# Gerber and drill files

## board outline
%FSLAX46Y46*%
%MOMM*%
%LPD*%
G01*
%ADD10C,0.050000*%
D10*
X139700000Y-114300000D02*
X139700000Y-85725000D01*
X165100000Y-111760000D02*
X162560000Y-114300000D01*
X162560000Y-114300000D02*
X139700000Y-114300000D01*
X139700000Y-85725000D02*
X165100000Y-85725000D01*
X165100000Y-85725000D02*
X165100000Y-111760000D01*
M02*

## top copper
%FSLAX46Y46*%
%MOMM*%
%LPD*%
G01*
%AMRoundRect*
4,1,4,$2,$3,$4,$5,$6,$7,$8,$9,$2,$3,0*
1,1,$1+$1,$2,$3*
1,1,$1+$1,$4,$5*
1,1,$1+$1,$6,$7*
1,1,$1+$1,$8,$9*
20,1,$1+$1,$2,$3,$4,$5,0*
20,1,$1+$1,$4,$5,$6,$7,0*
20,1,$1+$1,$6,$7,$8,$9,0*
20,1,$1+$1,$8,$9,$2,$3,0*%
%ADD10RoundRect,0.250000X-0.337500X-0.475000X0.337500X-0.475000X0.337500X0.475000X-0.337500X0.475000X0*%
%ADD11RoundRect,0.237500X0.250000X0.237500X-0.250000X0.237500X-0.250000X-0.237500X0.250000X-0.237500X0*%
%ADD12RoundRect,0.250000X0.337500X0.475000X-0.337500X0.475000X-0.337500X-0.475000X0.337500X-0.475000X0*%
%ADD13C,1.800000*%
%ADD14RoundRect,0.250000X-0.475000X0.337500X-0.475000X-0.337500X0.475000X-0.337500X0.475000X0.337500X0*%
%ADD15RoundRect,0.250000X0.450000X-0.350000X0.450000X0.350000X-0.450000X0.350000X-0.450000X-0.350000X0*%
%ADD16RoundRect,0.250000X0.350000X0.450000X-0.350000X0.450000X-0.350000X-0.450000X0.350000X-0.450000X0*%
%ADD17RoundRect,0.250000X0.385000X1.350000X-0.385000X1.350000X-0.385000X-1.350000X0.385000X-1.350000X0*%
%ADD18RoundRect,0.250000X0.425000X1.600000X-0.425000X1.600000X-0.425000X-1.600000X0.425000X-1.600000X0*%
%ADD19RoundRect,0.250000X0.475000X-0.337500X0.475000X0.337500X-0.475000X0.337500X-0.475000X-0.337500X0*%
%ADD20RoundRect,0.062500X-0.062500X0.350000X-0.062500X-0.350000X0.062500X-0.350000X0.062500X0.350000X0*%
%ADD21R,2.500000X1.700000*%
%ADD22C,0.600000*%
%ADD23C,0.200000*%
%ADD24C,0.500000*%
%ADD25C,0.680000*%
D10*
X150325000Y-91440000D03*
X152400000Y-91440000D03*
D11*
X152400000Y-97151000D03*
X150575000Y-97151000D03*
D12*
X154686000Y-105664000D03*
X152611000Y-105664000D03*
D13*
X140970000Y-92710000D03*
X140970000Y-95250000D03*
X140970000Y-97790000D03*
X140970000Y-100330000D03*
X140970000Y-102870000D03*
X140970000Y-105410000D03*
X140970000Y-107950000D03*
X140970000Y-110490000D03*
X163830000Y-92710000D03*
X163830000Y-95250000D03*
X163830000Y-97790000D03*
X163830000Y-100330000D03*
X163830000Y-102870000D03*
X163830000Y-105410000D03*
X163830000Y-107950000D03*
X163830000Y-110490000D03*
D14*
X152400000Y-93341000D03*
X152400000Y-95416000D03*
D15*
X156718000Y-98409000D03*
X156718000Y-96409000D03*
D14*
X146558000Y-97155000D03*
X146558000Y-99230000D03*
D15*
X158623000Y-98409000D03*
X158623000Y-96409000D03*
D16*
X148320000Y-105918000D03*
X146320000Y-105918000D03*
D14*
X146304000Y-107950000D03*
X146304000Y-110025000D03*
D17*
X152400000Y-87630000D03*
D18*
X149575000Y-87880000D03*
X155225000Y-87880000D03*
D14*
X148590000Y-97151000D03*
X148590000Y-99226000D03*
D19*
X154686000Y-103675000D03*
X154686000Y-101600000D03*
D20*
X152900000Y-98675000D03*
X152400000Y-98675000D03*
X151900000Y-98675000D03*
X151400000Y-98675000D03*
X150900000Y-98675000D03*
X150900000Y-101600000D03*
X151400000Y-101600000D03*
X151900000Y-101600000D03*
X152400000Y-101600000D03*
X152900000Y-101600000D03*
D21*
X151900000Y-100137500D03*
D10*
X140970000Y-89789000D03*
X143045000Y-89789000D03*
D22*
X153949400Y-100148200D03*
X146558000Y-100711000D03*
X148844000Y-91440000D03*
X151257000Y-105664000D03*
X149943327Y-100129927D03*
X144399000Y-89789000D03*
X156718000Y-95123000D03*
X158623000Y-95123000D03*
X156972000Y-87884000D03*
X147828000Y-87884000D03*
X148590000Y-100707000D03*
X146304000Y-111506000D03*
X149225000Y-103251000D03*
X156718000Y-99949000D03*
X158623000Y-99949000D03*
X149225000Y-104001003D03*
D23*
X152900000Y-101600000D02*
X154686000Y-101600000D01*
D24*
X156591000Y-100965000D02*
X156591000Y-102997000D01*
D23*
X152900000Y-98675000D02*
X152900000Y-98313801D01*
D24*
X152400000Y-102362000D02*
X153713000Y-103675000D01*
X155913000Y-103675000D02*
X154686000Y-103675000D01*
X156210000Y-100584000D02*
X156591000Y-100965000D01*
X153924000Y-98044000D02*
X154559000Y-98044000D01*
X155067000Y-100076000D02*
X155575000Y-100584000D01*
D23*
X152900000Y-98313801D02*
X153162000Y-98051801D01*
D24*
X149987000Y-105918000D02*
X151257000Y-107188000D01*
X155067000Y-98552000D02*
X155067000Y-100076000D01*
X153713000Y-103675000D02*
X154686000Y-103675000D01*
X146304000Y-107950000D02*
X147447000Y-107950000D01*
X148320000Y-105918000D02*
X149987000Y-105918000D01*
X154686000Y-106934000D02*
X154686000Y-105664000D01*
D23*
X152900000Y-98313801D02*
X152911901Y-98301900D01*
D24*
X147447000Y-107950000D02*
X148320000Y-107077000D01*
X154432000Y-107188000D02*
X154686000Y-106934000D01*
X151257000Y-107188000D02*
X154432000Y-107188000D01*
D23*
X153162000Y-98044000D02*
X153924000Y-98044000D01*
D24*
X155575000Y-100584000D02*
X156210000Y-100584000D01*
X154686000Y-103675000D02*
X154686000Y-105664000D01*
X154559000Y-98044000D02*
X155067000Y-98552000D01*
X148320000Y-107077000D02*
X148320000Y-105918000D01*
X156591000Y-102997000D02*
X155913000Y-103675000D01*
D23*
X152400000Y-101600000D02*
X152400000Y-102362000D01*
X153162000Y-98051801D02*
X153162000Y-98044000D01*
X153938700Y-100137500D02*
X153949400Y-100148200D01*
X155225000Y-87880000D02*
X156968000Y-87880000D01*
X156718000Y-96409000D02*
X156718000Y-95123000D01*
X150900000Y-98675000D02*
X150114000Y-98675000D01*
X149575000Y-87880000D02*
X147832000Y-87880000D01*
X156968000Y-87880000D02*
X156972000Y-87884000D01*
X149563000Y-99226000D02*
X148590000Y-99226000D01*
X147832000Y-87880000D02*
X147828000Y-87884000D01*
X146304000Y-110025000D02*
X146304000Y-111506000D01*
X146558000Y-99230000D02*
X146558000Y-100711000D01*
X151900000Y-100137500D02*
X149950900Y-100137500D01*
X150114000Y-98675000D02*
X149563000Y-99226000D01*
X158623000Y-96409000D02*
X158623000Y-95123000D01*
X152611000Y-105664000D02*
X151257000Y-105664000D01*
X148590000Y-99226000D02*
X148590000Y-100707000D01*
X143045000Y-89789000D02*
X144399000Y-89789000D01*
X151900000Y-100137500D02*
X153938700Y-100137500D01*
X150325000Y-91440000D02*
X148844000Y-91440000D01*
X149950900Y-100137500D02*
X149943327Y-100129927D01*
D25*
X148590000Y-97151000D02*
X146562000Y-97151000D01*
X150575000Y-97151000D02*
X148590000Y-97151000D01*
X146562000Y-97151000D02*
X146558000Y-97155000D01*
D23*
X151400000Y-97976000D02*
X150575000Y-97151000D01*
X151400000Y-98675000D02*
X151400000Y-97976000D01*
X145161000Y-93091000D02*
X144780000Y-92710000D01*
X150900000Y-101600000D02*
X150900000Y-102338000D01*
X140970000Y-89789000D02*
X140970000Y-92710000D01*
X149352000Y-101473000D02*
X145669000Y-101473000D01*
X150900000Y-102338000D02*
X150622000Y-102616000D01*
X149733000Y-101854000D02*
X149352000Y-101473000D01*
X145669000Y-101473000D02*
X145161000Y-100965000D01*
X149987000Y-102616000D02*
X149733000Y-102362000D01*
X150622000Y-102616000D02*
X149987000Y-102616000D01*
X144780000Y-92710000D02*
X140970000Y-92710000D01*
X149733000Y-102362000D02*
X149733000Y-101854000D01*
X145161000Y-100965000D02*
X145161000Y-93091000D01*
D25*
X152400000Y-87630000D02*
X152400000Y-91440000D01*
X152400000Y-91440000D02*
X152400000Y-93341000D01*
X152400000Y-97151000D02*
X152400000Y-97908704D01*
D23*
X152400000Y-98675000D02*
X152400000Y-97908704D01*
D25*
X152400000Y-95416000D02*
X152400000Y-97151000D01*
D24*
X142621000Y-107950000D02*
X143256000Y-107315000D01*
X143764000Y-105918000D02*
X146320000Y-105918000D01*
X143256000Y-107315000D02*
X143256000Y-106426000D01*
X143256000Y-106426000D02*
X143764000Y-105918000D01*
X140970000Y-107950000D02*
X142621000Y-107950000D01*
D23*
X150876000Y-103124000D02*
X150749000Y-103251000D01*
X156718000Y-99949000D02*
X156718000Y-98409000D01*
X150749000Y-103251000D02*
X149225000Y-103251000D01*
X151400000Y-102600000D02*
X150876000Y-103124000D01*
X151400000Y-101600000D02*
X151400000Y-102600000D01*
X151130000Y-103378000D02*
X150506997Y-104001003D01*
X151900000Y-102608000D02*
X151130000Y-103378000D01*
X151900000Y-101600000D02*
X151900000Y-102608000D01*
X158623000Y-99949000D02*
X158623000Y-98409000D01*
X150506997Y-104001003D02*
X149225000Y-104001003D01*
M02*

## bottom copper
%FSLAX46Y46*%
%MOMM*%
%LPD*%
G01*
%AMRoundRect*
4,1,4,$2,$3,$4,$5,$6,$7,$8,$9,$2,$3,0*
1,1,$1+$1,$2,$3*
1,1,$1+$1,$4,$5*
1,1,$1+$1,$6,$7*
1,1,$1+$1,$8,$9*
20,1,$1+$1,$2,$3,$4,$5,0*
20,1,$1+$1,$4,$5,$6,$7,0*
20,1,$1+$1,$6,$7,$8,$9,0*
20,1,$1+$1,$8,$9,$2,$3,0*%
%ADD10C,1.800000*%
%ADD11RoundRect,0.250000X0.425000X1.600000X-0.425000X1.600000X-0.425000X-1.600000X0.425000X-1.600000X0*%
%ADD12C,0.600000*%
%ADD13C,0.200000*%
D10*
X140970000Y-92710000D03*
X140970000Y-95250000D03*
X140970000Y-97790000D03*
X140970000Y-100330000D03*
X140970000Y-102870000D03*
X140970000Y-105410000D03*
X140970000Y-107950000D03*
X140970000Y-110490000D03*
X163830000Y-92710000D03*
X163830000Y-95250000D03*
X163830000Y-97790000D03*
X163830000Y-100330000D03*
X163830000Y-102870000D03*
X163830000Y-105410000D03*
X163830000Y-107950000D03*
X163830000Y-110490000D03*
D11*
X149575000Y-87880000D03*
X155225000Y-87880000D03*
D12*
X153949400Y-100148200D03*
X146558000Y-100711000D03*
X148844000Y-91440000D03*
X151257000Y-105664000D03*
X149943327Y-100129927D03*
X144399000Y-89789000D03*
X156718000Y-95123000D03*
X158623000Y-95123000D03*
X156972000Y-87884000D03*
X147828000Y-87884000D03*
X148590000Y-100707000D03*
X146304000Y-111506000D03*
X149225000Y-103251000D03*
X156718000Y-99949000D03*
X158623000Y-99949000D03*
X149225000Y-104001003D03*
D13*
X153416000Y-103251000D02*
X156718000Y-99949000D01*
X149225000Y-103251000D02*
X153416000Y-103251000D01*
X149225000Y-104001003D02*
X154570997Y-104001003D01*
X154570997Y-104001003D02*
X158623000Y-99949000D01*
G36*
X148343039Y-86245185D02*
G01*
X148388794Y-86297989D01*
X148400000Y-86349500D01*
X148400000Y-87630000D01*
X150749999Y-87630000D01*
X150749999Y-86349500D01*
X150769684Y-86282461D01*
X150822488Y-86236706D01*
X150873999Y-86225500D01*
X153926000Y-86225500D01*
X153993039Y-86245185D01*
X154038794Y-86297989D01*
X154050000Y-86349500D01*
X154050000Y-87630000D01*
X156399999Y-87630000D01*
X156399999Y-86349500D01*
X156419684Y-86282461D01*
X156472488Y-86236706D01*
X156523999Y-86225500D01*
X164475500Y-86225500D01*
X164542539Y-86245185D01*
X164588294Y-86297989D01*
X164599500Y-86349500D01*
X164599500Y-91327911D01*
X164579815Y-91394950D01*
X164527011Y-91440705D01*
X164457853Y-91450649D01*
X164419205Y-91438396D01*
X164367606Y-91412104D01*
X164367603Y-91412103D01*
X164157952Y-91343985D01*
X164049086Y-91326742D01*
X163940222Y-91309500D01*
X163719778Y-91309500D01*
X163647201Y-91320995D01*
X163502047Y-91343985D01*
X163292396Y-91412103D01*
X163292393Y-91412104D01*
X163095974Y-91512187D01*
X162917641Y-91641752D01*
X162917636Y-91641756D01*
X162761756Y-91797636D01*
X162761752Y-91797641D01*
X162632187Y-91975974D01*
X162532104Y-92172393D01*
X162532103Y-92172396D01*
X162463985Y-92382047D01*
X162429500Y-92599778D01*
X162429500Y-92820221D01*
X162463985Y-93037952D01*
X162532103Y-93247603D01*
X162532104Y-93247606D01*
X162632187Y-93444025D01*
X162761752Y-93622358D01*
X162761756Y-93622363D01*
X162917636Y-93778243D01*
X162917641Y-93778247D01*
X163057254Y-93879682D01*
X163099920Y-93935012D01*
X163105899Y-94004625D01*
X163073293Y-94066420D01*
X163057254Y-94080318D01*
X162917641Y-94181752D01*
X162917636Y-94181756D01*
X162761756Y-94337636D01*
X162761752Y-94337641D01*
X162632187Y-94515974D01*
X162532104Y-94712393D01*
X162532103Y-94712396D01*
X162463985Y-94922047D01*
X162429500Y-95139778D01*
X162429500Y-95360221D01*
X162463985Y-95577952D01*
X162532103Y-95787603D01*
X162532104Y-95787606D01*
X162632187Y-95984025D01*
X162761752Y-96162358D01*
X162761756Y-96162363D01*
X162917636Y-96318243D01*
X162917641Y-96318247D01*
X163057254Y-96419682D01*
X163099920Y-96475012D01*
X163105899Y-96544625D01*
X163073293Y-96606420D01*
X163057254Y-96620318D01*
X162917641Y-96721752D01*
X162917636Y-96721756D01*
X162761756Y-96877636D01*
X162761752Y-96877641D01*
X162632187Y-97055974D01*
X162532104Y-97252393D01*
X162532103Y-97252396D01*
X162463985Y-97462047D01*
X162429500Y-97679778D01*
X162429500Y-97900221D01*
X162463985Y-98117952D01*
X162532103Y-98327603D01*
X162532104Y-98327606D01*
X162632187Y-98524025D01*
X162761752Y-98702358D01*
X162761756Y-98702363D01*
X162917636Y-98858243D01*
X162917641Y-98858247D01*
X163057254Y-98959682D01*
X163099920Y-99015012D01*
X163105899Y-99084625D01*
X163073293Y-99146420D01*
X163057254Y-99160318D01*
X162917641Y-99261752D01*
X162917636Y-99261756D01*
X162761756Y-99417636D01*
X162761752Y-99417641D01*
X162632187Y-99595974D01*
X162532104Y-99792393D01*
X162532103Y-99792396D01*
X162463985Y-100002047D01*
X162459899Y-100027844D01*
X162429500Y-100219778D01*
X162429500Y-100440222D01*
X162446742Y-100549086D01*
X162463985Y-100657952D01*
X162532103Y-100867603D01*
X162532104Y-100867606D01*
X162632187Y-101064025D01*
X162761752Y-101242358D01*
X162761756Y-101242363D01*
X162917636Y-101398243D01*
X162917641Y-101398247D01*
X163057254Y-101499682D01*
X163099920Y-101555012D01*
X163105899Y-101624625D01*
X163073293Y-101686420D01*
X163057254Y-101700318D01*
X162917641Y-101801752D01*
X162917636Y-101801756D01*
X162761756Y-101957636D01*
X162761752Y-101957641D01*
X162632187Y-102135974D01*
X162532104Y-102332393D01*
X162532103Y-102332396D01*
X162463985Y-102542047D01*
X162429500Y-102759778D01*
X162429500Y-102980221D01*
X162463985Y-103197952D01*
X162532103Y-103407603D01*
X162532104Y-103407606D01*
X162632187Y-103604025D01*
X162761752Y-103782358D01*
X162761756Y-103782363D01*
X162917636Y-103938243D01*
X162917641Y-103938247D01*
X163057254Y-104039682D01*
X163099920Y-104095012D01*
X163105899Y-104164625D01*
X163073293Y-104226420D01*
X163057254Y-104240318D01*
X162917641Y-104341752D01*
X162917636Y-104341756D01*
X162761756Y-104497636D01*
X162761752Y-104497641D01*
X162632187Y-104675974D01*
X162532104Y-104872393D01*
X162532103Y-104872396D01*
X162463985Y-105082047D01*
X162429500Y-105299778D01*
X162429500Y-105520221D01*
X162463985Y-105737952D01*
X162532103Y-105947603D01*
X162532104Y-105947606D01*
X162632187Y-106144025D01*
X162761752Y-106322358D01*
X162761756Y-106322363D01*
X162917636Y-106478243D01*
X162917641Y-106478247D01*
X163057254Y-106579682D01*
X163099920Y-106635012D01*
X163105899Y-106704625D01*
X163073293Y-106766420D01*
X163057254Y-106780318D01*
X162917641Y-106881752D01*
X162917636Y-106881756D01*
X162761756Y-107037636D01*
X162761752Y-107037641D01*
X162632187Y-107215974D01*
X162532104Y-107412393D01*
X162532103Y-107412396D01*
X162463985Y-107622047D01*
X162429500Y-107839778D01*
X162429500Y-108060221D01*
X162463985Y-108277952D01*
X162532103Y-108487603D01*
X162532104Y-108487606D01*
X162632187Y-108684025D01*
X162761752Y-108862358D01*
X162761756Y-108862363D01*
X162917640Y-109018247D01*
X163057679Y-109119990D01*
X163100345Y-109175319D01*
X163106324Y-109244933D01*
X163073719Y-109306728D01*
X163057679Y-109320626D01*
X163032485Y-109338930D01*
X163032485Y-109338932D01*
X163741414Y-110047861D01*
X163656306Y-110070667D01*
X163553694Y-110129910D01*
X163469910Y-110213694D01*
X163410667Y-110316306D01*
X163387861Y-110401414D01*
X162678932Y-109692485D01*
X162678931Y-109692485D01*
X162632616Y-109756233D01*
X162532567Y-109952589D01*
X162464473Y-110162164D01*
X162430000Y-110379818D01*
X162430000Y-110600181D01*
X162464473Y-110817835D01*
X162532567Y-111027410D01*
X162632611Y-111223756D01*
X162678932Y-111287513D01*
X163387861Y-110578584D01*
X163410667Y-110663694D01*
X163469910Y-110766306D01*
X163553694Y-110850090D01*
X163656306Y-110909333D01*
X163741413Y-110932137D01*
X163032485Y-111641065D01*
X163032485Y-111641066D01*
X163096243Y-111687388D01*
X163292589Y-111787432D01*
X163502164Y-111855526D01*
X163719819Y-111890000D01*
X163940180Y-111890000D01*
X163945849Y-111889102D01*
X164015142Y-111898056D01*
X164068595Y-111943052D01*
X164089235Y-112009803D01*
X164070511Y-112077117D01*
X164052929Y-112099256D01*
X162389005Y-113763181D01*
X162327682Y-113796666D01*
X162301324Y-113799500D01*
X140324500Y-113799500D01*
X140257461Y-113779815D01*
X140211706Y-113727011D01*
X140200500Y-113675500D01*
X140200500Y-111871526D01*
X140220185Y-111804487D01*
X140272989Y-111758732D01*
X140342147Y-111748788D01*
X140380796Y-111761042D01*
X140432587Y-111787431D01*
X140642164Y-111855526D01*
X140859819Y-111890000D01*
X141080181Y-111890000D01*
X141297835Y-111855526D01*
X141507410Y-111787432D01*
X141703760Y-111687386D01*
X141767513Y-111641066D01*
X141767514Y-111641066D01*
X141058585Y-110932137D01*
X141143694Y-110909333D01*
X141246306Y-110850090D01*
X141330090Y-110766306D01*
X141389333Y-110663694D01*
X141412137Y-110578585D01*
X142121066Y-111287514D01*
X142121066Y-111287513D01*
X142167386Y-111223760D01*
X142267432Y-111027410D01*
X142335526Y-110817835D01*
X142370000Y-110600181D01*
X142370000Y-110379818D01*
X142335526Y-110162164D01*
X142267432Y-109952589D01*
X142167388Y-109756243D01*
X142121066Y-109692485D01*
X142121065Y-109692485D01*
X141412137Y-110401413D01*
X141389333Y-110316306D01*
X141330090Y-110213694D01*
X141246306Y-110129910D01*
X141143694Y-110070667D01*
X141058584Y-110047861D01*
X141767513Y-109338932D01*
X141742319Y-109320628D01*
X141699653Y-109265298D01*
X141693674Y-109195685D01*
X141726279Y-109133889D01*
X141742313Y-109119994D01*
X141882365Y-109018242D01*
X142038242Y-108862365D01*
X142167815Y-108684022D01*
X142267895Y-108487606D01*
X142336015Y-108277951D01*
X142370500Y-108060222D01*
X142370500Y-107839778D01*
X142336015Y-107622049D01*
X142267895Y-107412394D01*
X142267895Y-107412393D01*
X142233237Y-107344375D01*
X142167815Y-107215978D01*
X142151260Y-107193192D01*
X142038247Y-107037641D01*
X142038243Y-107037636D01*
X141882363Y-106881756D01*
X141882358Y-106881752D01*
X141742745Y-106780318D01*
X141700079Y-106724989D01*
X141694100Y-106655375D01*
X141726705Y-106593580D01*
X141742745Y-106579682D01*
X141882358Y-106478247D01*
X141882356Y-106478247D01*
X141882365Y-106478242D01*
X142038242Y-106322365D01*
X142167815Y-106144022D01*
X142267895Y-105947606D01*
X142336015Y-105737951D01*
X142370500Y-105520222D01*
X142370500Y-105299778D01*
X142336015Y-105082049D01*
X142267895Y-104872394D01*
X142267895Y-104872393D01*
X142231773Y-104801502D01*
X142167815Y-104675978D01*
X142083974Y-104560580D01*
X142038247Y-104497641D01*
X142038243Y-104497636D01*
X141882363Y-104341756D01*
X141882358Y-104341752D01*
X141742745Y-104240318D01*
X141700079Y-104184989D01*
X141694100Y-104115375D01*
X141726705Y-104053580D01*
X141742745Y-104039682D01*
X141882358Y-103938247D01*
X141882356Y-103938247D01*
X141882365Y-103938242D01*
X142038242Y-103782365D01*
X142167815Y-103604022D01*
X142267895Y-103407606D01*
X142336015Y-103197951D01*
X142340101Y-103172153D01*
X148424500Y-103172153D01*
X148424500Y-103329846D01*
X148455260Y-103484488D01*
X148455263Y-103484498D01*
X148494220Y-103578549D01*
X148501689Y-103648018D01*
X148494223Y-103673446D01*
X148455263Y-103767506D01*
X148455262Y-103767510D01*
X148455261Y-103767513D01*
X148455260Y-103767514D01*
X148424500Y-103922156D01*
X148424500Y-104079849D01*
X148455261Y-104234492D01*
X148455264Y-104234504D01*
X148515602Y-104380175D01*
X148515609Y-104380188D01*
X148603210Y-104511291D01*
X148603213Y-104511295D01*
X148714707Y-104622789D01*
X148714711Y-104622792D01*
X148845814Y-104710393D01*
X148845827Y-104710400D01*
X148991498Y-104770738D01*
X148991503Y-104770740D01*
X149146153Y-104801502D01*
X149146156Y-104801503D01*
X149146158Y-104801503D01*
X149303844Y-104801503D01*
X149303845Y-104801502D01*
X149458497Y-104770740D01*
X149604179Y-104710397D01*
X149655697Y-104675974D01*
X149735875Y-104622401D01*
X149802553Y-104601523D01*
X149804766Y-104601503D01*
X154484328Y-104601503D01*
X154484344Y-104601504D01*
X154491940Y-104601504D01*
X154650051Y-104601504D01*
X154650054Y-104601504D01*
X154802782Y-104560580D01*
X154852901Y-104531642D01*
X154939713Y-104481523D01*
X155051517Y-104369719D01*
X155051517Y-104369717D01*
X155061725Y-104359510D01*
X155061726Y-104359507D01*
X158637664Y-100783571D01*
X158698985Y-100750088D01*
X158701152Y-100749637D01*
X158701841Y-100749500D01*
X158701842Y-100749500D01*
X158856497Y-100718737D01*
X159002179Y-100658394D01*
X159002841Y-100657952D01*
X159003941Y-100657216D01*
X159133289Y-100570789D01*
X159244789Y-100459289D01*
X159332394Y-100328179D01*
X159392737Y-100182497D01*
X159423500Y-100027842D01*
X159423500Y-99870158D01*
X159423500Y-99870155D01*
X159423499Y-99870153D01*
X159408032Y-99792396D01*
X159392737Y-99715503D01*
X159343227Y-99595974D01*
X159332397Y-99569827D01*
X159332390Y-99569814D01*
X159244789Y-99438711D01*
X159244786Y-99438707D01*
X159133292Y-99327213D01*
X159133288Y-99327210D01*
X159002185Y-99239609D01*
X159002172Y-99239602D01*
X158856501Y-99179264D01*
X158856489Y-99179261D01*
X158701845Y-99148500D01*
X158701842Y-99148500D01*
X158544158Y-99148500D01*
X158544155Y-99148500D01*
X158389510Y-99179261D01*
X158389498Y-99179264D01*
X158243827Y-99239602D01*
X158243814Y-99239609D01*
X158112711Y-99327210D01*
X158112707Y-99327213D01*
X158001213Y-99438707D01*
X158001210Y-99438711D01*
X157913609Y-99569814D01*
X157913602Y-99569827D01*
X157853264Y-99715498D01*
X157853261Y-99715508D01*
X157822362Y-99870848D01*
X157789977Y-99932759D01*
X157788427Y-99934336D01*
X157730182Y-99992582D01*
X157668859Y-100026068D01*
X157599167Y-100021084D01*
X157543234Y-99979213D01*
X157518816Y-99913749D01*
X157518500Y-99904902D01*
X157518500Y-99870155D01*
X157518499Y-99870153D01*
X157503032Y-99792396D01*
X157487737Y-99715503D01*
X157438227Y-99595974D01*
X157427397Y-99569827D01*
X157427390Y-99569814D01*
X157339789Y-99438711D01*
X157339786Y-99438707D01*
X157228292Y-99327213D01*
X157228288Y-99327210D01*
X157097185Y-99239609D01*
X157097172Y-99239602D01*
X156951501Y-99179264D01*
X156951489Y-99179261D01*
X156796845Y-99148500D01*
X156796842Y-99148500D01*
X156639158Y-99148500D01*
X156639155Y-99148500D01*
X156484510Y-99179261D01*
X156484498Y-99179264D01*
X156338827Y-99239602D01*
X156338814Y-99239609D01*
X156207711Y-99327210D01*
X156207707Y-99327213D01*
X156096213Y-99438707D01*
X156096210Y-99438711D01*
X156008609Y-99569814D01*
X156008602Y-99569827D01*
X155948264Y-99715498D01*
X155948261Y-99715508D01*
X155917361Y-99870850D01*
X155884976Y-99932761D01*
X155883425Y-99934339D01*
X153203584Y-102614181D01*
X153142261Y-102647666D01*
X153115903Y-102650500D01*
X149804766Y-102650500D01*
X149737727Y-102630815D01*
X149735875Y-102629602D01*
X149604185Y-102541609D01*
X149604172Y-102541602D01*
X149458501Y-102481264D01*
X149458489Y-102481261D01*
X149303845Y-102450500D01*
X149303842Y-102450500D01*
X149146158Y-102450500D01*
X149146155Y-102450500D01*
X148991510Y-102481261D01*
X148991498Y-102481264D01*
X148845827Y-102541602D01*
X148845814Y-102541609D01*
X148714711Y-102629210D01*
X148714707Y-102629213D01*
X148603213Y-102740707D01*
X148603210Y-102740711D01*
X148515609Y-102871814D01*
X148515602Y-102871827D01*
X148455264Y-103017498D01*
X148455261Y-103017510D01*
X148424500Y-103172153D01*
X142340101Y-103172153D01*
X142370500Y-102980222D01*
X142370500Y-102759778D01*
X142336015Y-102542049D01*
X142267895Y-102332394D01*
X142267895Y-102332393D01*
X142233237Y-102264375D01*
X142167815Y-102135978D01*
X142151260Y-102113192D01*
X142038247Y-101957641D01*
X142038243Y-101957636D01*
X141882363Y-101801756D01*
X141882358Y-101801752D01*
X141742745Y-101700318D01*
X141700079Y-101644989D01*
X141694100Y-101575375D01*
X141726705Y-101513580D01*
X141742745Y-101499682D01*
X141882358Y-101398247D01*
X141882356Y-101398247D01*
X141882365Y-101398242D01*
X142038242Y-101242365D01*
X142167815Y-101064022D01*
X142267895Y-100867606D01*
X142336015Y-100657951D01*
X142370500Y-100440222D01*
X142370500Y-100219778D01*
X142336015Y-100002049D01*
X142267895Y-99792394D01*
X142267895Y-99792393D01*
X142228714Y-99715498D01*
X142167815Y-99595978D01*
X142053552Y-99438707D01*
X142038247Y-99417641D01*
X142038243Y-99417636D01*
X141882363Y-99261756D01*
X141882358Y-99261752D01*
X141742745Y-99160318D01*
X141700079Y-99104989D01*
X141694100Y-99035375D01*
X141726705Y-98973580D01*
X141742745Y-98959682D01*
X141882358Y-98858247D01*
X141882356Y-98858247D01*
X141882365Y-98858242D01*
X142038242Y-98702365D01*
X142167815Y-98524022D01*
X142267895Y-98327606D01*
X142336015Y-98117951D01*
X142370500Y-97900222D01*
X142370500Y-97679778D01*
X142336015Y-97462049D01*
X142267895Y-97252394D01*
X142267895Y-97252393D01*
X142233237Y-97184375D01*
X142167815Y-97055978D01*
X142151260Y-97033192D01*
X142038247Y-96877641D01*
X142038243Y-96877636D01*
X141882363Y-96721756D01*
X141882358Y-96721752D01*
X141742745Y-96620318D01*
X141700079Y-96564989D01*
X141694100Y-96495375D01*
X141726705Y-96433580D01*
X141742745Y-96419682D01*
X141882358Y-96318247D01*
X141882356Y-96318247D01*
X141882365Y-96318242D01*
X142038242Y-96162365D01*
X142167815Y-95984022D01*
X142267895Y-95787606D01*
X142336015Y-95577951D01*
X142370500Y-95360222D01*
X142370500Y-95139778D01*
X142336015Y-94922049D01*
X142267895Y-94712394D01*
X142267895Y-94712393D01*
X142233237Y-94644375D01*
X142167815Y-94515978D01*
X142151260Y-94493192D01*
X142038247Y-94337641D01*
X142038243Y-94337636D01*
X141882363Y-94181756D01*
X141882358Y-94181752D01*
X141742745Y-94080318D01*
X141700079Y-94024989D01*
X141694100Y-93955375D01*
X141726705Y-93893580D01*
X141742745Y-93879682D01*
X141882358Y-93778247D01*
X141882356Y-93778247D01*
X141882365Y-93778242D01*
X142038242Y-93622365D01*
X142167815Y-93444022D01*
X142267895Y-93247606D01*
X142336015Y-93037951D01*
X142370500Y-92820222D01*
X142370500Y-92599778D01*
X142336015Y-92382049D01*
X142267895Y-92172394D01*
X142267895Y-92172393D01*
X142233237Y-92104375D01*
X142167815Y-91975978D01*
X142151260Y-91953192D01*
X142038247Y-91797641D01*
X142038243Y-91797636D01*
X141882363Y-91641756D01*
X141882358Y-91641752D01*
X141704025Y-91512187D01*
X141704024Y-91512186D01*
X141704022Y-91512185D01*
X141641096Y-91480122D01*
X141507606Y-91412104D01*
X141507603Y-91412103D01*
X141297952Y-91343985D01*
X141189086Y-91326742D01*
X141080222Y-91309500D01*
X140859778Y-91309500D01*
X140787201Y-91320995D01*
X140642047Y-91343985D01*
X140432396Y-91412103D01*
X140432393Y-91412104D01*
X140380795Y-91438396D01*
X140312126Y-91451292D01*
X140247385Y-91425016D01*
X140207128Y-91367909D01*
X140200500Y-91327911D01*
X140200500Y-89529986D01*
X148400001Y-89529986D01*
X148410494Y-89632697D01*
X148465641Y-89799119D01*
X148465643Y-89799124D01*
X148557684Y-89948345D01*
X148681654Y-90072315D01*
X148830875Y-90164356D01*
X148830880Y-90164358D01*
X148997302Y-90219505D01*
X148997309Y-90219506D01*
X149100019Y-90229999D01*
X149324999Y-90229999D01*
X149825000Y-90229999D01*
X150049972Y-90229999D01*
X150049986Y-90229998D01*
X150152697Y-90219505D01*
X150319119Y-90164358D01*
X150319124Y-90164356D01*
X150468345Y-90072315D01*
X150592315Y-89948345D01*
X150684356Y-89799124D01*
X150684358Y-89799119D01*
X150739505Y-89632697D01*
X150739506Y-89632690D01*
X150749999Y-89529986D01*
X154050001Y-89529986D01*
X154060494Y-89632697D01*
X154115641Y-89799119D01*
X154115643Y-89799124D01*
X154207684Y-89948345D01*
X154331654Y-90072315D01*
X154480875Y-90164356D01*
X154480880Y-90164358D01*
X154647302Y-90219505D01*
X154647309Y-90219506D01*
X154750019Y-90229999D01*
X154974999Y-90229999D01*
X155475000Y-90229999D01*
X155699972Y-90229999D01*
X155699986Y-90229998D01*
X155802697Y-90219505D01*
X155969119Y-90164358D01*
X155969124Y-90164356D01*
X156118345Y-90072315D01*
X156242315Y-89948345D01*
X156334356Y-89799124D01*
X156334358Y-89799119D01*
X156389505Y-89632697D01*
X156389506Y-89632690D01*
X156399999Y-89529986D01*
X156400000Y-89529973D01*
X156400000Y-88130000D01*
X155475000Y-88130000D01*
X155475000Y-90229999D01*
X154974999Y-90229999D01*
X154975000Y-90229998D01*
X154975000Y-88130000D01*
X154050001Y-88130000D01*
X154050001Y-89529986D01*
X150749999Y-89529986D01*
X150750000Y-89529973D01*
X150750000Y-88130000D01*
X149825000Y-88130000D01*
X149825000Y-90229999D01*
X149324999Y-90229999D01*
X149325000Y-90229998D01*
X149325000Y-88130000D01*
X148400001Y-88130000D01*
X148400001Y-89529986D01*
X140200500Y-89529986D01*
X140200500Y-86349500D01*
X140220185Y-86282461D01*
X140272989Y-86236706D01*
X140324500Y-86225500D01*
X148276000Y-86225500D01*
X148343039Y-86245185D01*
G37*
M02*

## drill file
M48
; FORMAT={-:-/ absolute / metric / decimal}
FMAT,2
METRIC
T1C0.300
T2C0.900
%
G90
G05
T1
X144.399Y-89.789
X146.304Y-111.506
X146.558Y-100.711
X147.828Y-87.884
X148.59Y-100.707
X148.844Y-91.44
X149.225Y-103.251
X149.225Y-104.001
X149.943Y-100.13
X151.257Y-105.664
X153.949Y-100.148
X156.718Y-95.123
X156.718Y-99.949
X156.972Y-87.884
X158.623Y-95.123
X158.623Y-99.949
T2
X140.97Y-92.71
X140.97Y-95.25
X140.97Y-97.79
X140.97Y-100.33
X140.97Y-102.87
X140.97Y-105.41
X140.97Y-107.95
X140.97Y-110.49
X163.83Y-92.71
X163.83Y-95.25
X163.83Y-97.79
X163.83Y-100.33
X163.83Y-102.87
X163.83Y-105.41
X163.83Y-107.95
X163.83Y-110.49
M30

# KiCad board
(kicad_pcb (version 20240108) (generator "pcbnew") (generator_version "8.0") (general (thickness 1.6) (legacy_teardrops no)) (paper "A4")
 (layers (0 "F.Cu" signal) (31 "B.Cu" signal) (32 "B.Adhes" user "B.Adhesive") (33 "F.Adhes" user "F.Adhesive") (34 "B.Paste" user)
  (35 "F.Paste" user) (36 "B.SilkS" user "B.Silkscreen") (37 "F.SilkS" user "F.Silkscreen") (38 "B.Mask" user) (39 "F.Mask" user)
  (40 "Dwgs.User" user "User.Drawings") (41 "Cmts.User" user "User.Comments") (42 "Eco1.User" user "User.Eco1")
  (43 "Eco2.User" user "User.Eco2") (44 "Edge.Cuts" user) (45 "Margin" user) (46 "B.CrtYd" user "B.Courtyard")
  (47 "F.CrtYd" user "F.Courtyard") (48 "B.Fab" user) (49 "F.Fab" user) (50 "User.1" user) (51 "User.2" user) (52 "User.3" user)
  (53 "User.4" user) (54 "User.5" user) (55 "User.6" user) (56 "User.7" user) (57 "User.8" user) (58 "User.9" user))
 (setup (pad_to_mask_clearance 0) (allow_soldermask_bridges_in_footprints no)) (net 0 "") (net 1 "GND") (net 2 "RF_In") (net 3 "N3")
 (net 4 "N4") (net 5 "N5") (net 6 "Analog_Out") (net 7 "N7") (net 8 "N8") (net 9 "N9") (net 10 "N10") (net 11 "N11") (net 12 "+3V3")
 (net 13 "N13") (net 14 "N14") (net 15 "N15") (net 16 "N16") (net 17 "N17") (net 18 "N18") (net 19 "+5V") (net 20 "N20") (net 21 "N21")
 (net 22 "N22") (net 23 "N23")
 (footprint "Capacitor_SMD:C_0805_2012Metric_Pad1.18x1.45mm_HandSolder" (layer "F.Cu") (at 151.3625 91.44)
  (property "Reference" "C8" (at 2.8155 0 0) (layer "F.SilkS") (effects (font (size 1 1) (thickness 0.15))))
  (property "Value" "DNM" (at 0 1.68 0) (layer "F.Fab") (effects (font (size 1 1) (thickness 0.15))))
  (pad "1" smd roundrect (at -1.0375 0) (size 1.175 1.45) (layers "F.Cu" "F.Paste" "F.Mask") (roundrect_rratio 0.212766) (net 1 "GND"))
  (pad "2" smd roundrect (at 1.0375 0) (size 1.175 1.45) (layers "F.Cu" "F.Paste" "F.Mask") (roundrect_rratio 0.212766) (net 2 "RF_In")))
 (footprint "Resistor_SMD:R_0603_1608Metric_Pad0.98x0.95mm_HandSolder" (layer "F.Cu") (at 151.4875 97.151 180)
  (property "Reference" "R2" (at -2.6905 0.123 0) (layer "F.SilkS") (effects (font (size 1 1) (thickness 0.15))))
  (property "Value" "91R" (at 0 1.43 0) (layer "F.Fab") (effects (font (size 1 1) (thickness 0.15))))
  (pad "1" smd roundrect (at -0.9125 0 180) (size 0.975 0.95) (layers "F.Cu" "F.Paste" "F.Mask") (roundrect_rratio 0.25) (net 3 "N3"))
  (pad "2" smd roundrect (at 0.9125 0 180) (size 0.975 0.95) (layers "F.Cu" "F.Paste" "F.Mask") (roundrect_rratio 0.25) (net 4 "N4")))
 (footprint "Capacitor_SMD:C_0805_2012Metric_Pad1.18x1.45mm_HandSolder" (layer "F.Cu") (at 153.6485 105.664 180)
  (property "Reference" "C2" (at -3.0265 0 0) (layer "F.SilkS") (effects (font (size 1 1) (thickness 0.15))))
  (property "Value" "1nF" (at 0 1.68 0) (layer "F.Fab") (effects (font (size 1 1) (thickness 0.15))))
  (pad "1" smd roundrect (at -1.0375 0 180) (size 1.175 1.45) (layers "F.Cu" "F.Paste" "F.Mask") (roundrect_rratio 0.212766) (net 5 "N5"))
  (pad "2" smd roundrect (at 1.0375 0 180) (size 1.175 1.45) (layers "F.Cu" "F.Paste" "F.Mask") (roundrect_rratio 0.212766) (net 1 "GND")))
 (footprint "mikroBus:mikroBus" (layer "F.Cu") (at 152.4 106.68)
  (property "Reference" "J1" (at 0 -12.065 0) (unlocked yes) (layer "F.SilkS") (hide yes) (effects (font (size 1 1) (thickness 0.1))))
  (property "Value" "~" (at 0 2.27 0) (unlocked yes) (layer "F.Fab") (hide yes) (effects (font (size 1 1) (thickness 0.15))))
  (pad "1" thru_hole circle (at -11.43 -13.97) (size 1.8 1.8) (drill 0.9) (layers "*.Cu" "*.Mask") (remove_unused_layers no)
   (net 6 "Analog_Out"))
  (pad "2" thru_hole circle (at -11.43 -11.43) (size 1.8 1.8) (drill 0.9) (layers "*.Cu" "*.Mask") (remove_unused_layers no) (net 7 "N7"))
  (pad "3" thru_hole circle (at -11.43 -8.89) (size 1.8 1.8) (drill 0.9) (layers "*.Cu" "*.Mask") (remove_unused_layers no) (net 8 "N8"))
  (pad "4" thru_hole circle (at -11.43 -6.35) (size 1.8 1.8) (drill 0.9) (layers "*.Cu" "*.Mask") (remove_unused_layers no) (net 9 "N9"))
  (pad "5" thru_hole circle (at -11.43 -3.81) (size 1.8 1.8) (drill 0.9) (layers "*.Cu" "*.Mask") (remove_unused_layers no) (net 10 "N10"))
  (pad "6" thru_hole circle (at -11.43 -1.27) (size 1.8 1.8) (drill 0.9) (layers "*.Cu" "*.Mask") (remove_unused_layers no) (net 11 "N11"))
  (pad "7" thru_hole circle (at -11.43 1.27) (size 1.8 1.8) (drill 0.9) (layers "*.Cu" "*.Mask") (remove_unused_layers no) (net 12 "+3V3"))
  (pad "8" thru_hole circle (at -11.43 3.81) (size 1.8 1.8) (drill 0.9) (layers "*.Cu" "*.Mask") (remove_unused_layers no) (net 1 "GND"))
  (pad "9" thru_hole circle (at 11.43 -13.97) (size 1.8 1.8) (drill 0.9) (layers "*.Cu" "*.Mask") (remove_unused_layers no) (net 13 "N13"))
  (pad "10" thru_hole circle (at 11.43 -11.43) (size 1.8 1.8) (drill 0.9) (layers "*.Cu" "*.Mask") (remove_unused_layers no) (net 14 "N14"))
  (pad "11" thru_hole circle (at 11.43 -8.89) (size 1.8 1.8) (drill 0.9) (layers "*.Cu" "*.Mask") (remove_unused_layers no) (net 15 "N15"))
  (pad "12" thru_hole circle (at 11.43 -6.35) (size 1.8 1.8) (drill 0.9) (layers "*.Cu" "*.Mask") (remove_unused_layers no) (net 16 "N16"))
  (pad "13" thru_hole circle (at 11.43 -3.81) (size 1.8 1.8) (drill 0.9) (layers "*.Cu" "*.Mask") (remove_unused_layers no) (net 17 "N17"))
  (pad "14" thru_hole circle (at 11.43 -1.27) (size 1.8 1.8) (drill 0.9) (layers "*.Cu" "*.Mask") (remove_unused_layers no) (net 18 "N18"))
  (pad "15" thru_hole circle (at 11.43 1.27) (size 1.8 1.8) (drill 0.9) (layers "*.Cu" "*.Mask") (remove_unused_layers no) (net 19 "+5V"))
  (pad "16" thru_hole circle (at 11.43 3.81) (size 1.8 1.8) (drill 0.9) (layers "*.Cu" "*.Mask") (remove_unused_layers no) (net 1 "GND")))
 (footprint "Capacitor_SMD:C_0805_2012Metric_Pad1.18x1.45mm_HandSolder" (layer "F.Cu") (at 152.4 94.3785 -90)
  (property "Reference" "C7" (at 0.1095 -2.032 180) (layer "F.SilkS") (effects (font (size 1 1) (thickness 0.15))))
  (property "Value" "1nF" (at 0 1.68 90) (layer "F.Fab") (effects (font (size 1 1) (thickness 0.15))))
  (pad "1" smd roundrect (at -1.0375 0 270) (size 1.175 1.45) (layers "F.Cu" "F.Paste" "F.Mask") (roundrect_rratio 0.212766) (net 2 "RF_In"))
  (pad "2" smd roundrect (at 1.0375 0 270) (size 1.175 1.45) (layers "F.Cu" "F.Paste" "F.Mask") (roundrect_rratio 0.212766) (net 3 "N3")))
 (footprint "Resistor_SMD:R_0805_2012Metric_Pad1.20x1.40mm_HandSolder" (layer "F.Cu") (at 156.718 97.409 90)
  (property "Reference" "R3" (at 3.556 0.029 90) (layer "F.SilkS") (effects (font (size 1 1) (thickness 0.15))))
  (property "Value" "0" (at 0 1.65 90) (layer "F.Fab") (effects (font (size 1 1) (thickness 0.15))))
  (pad "1" smd roundrect (at -1 0 90) (size 1.2 1.4) (layers "F.Cu" "F.Paste" "F.Mask") (roundrect_rratio 0.208333) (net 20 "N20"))
  (pad "2" smd roundrect (at 1 0 90) (size 1.2 1.4) (layers "F.Cu" "F.Paste" "F.Mask") (roundrect_rratio 0.208333) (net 1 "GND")))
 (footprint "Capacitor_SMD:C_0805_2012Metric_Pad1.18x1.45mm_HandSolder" (layer "F.Cu") (at 146.558 98.1925 -90)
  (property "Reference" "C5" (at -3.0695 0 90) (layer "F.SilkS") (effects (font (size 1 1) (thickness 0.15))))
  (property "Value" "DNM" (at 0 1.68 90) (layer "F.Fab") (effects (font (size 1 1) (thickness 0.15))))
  (pad "1" smd roundrect (at -1.0375 0 270) (size 1.175 1.45) (layers "F.Cu" "F.Paste" "F.Mask") (roundrect_rratio 0.212766) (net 4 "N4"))
  (pad "2" smd roundrect (at 1.0375 0 270) (size 1.175 1.45) (layers "F.Cu" "F.Paste" "F.Mask") (roundrect_rratio 0.212766) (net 1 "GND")))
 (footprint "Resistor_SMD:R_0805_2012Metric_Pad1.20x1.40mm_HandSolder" (layer "F.Cu") (at 158.623 97.409 90)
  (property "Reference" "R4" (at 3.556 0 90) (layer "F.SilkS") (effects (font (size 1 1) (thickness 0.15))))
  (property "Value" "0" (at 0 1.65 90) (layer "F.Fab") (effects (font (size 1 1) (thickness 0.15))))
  (pad "1" smd roundrect (at -1 0 90) (size 1.2 1.4) (layers "F.Cu" "F.Paste" "F.Mask") (roundrect_rratio 0.208333) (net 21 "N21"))
  (pad "2" smd roundrect (at 1 0 90) (size 1.2 1.4) (layers "F.Cu" "F.Paste" "F.Mask") (roundrect_rratio 0.208333) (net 1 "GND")))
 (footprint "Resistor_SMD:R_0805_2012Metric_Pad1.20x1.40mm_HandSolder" (layer "F.Cu") (at 147.32 105.918 180)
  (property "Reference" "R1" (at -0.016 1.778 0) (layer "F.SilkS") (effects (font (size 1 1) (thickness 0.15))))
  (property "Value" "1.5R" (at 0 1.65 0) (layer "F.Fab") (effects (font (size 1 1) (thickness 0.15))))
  (pad "1" smd roundrect (at -1 0 180) (size 1.2 1.4) (layers "F.Cu" "F.Paste" "F.Mask") (roundrect_rratio 0.208333) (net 5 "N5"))
  (pad "2" smd roundrect (at 1 0 180) (size 1.2 1.4) (layers "F.Cu" "F.Paste" "F.Mask") (roundrect_rratio 0.208333) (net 12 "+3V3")))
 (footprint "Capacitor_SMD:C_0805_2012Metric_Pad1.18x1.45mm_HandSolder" (layer "F.Cu") (at 146.304 108.9875 -90)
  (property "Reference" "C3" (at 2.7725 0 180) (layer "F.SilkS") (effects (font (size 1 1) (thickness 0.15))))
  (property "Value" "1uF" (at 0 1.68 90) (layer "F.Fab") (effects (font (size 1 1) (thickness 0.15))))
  (pad "1" smd roundrect (at -1.0375 0 270) (size 1.175 1.45) (layers "F.Cu" "F.Paste" "F.Mask") (roundrect_rratio 0.212766) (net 5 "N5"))
  (pad "2" smd roundrect (at 1.0375 0 270) (size 1.175 1.45) (layers "F.Cu" "F.Paste" "F.Mask") (roundrect_rratio 0.212766) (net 1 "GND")))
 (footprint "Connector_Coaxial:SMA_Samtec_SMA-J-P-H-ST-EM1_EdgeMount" (layer "F.Cu") (at 152.4 87.63 90)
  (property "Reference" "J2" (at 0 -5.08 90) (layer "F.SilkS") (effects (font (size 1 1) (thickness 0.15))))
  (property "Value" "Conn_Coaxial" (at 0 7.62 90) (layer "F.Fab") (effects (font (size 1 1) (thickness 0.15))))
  (pad "1" smd roundrect (at 0 0 180) (size 1.27 3.2) (layers "F.Cu" "F.Mask") (roundrect_rratio 0.1968503937) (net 2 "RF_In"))
  (pad "2" smd roundrect (at -0.25 -2.825 180) (size 1.35 3.7) (layers "F.Cu" "F.Mask") (roundrect_rratio 0.1851851852) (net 1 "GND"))
  (pad "2" smd roundrect (at -0.25 -2.825 180) (size 1.35 3.7) (layers "B.Cu" "B.Mask") (roundrect_rratio 0.1851851852) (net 1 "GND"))
  (pad "2" smd roundrect (at -0.25 2.825 180) (size 1.35 3.7) (layers "F.Cu" "F.Mask") (roundrect_rratio 0.1851851852) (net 1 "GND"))
  (pad "2" smd roundrect (at -0.25 2.825 180) (size 1.35 3.7) (layers "B.Cu" "B.Mask") (roundrect_rratio 0.1851851852) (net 1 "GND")))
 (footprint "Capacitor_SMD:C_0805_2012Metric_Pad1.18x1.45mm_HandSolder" (layer "F.Cu") (at 148.59 98.1885 -90)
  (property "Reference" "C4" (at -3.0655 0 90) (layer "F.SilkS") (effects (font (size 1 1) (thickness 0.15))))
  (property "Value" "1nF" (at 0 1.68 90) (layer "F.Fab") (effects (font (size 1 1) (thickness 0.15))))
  (pad "1" smd roundrect (at -1.0375 0 270) (size 1.175 1.45) (layers "F.Cu" "F.Paste" "F.Mask") (roundrect_rratio 0.212766) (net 4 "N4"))
  (pad "2" smd roundrect (at 1.0375 0 270) (size 1.175 1.45) (layers "F.Cu" "F.Paste" "F.Mask") (roundrect_rratio 0.212766) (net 1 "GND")))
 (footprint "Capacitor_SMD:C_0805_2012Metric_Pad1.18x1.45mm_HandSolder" (layer "F.Cu") (at 154.686 102.6375 90)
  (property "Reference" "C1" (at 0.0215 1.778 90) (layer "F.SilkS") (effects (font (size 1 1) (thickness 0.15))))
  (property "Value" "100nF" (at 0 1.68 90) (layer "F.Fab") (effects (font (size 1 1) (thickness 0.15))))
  (pad "1" smd roundrect (at -1.0375 0 90) (size 1.175 1.45) (layers "F.Cu" "F.Paste" "F.Mask") (roundrect_rratio 0.212766) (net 5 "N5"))
  (pad "2" smd roundrect (at 1.0375 0 90) (size 1.175 1.45) (layers "F.Cu" "F.Paste" "F.Mask") (roundrect_rratio 0.212766) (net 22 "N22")))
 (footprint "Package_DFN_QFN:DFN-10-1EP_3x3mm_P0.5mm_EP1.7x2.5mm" (layer "F.Cu") (at 151.9 100.1375 -90)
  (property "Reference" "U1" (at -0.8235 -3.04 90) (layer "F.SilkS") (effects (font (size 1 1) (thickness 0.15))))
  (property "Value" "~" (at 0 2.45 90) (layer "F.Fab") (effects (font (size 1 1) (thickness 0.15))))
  (pad "" smd roundrect (at -0.425 -0.625 270) (size 0.69 1.01) (layers "F.Paste") (roundrect_rratio 0.25))
  (pad "" smd roundrect (at -0.425 0.625 270) (size 0.69 1.01) (layers "F.Paste") (roundrect_rratio 0.25))
  (pad "" smd roundrect (at 0.425 -0.625 270) (size 0.69 1.01) (layers "F.Paste") (roundrect_rratio 0.25))
  (pad "" smd roundrect (at 0.425 0.625 270) (size 0.69 1.01) (layers "F.Paste") (roundrect_rratio 0.25))
  (pad "1" smd roundrect (at -1.4625 -1 270) (size 0.825 0.25) (layers "F.Cu" "F.Paste" "F.Mask") (roundrect_rratio 0.25) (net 5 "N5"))
  (pad "2" smd roundrect (at -1.4625 -0.5 270) (size 0.825 0.25) (layers "F.Cu" "F.Paste" "F.Mask") (roundrect_rratio 0.25) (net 3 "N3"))
  (pad "3" smd roundrect (at -1.4625 0 270) (size 0.825 0.25) (layers "F.Cu" "F.Paste" "F.Mask") (roundrect_rratio 0.25) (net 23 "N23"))
  (pad "4" smd roundrect (at -1.4625 0.5 270) (size 0.825 0.25) (layers "F.Cu" "F.Paste" "F.Mask") (roundrect_rratio 0.25) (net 4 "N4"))
  (pad "5" smd roundrect (at -1.4625 1 270) (size 0.825 0.25) (layers "F.Cu" "F.Paste" "F.Mask") (roundrect_rratio 0.25) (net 1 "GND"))
  (pad "6" smd roundrect (at 1.4625 1 270) (size 0.825 0.25) (layers "F.Cu" "F.Paste" "F.Mask") (roundrect_rratio 0.25) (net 6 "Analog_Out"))
  (pad "7" smd roundrect (at 1.4625 0.5 270) (size 0.825 0.25) (layers "F.Cu" "F.Paste" "F.Mask") (roundrect_rratio 0.25) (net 20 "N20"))
  (pad "8" smd roundrect (at 1.4625 0 270) (size 0.825 0.25) (layers "F.Cu" "F.Paste" "F.Mask") (roundrect_rratio 0.25) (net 21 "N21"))
  (pad "9" smd roundrect (at 1.4625 -0.5 270) (size 0.825 0.25) (layers "F.Cu" "F.Paste" "F.Mask") (roundrect_rratio 0.25) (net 5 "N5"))
  (pad "10" smd roundrect (at 1.4625 -1 270) (size 0.825 0.25) (layers "F.Cu" "F.Paste" "F.Mask") (roundrect_rratio 0.25) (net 22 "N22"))
  (pad "11" smd rect (at 0 0 270) (size 1.7 2.5) (layers "F.Cu" "F.Mask") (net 1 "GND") (zone_connect 2)))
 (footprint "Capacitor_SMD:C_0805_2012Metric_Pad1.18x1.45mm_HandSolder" (layer "F.Cu") (at 142.0075 89.789)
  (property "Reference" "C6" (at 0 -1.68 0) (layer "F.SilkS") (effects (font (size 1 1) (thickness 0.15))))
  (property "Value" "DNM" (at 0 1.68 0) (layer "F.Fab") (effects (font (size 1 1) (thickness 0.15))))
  (pad "1" smd roundrect (at -1.0375 0) (size 1.175 1.45) (layers "F.Cu" "F.Paste" "F.Mask") (roundrect_rratio 0.212766)
   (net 6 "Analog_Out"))
  (pad "2" smd roundrect (at 1.0375 0) (size 1.175 1.45) (layers "F.Cu" "F.Paste" "F.Mask") (roundrect_rratio 0.212766) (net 1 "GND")))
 (gr_line (start 139.7 114.3) (end 139.7 85.725) (stroke (width 0.05) (type default)) (layer "Edge.Cuts"))
 (gr_line (start 165.1 111.76) (end 162.56 114.3) (stroke (width 0.05) (type default)) (layer "Edge.Cuts"))
 (gr_line (start 162.56 114.3) (end 139.7 114.3) (stroke (width 0.05) (type default)) (layer "Edge.Cuts"))
 (gr_line (start 139.7 85.725) (end 165.1 85.725) (stroke (width 0.05) (type default)) (layer "Edge.Cuts"))
 (gr_line (start 165.1 85.725) (end 165.1 111.76) (stroke (width 0.05) (type default)) (layer "Edge.Cuts"))
 (segment (start 152.9 101.6) (end 154.686 101.6) (width 0.2) (layer "F.Cu") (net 22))
 (segment (start 156.591 100.965) (end 156.591 102.997) (width 0.5) (layer "F.Cu") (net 5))
 (segment (start 152.9 98.675) (end 152.9 98.313801) (width 0.2) (layer "F.Cu") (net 5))
 (segment (start 152.4 102.362) (end 153.713 103.675) (width 0.5) (layer "F.Cu") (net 5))
 (segment (start 155.913 103.675) (end 154.686 103.675) (width 0.5) (layer "F.Cu") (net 5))
 (segment (start 156.21 100.584) (end 156.591 100.965) (width 0.5) (layer "F.Cu") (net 5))
 (segment (start 153.924 98.044) (end 154.559 98.044) (width 0.5) (layer "F.Cu") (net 5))
 (segment (start 155.067 100.076) (end 155.575 100.584) (width 0.5) (layer "F.Cu") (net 5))
 (segment (start 152.9 98.313801) (end 153.162 98.051801) (width 0.2) (layer "F.Cu") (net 5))
 (segment (start 149.987 105.918) (end 151.257 107.188) (width 0.5) (layer "F.Cu") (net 5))
 (segment (start 155.067 98.552) (end 155.067 100.076) (width 0.5) (layer "F.Cu") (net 5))
 (segment (start 153.713 103.675) (end 154.686 103.675) (width 0.5) (layer "F.Cu") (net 5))
 (segment (start 146.304 107.95) (end 147.447 107.95) (width 0.5) (layer "F.Cu") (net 5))
 (segment (start 148.32 105.918) (end 149.987 105.918) (width 0.5) (layer "F.Cu") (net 5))
 (segment (start 154.686 106.934) (end 154.686 105.664) (width 0.5) (layer "F.Cu") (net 5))
 (segment (start 152.9 98.313801) (end 152.911901 98.3019) (width 0.2) (layer "F.Cu") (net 5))
 (segment (start 147.447 107.95) (end 148.32 107.077) (width 0.5) (layer "F.Cu") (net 5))
 (segment (start 154.432 107.188) (end 154.686 106.934) (width 0.5) (layer "F.Cu") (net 5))
 (segment (start 151.257 107.188) (end 154.432 107.188) (width 0.5) (layer "F.Cu") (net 5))
 (segment (start 153.162 98.044) (end 153.924 98.044) (width 0.2) (layer "F.Cu") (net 5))
 (segment (start 155.575 100.584) (end 156.21 100.584) (width 0.5) (layer "F.Cu") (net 5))
 (segment (start 154.686 103.675) (end 154.686 105.664) (width 0.5) (layer "F.Cu") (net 5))
 (segment (start 154.559 98.044) (end 155.067 98.552) (width 0.5) (layer "F.Cu") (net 5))
 (segment (start 148.32 107.077) (end 148.32 105.918) (width 0.5) (layer "F.Cu") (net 5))
 (segment (start 156.591 102.997) (end 155.913 103.675) (width 0.5) (layer "F.Cu") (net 5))
 (segment (start 152.4 101.6) (end 152.4 102.362) (width 0.2) (layer "F.Cu") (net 5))
 (segment (start 153.162 98.051801) (end 153.162 98.044) (width 0.2) (layer "F.Cu") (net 5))
 (segment (start 153.9387 100.1375) (end 153.9494 100.1482) (width 0.2) (layer "F.Cu") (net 1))
 (segment (start 155.225 87.88) (end 156.968 87.88) (width 0.2) (layer "F.Cu") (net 1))
 (segment (start 156.718 96.409) (end 156.718 95.123) (width 0.2) (layer "F.Cu") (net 1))
 (segment (start 150.9 98.675) (end 150.114 98.675) (width 0.2) (layer "F.Cu") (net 1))
 (segment (start 149.575 87.88) (end 147.832 87.88) (width 0.2) (layer "F.Cu") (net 1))
 (segment (start 156.968 87.88) (end 156.972 87.884) (width 0.2) (layer "F.Cu") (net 1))
 (segment (start 149.563 99.226) (end 148.59 99.226) (width 0.2) (layer "F.Cu") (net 1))
 (segment (start 147.832 87.88) (end 147.828 87.884) (width 0.2) (layer "F.Cu") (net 1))
 (segment (start 146.304 110.025) (end 146.304 111.506) (width 0.2) (layer "F.Cu") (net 1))
 (segment (start 146.558 99.23) (end 146.558 100.711) (width 0.2) (layer "F.Cu") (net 1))
 (segment (start 151.9 100.1375) (end 149.9509 100.1375) (width 0.2) (layer "F.Cu") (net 1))
 (segment (start 150.114 98.675) (end 149.563 99.226) (width 0.2) (layer "F.Cu") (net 1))
 (segment (start 158.623 96.409) (end 158.623 95.123) (width 0.2) (layer "F.Cu") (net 1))
 (segment (start 152.611 105.664) (end 151.257 105.664) (width 0.2) (layer "F.Cu") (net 1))
 (segment (start 148.59 99.226) (end 148.59 100.707) (width 0.2) (layer "F.Cu") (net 1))
 (segment (start 143.045 89.789) (end 144.399 89.789) (width 0.2) (layer "F.Cu") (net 1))
 (segment (start 151.9 100.1375) (end 153.9387 100.1375) (width 0.2) (layer "F.Cu") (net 1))
 (segment (start 150.325 91.44) (end 148.844 91.44) (width 0.2) (layer "F.Cu") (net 1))
 (segment (start 149.9509 100.1375) (end 149.943327 100.129927) (width 0.2) (layer "F.Cu") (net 1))
 (via (at 153.9494 100.1482) (size 0.6) (drill 0.3) (layers "F.Cu" "B.Cu") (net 1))
 (via (at 146.558 100.711) (size 0.6) (drill 0.3) (layers "F.Cu" "B.Cu") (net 1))
 (via (at 148.844 91.44) (size 0.6) (drill 0.3) (layers "F.Cu" "B.Cu") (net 1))
 (via (at 151.257 105.664) (size 0.6) (drill 0.3) (layers "F.Cu" "B.Cu") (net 1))
 (via (at 149.943327 100.129927) (size 0.6) (drill 0.3) (layers "F.Cu" "B.Cu") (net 1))
 (via (at 144.399 89.789) (size 0.6) (drill 0.3) (layers "F.Cu" "B.Cu") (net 1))
 (via (at 156.718 95.123) (size 0.6) (drill 0.3) (layers "F.Cu" "B.Cu") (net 1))
 (via (at 158.623 95.123) (size 0.6) (drill 0.3) (layers "F.Cu" "B.Cu") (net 1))
 (via (at 156.972 87.884) (size 0.6) (drill 0.3) (layers "F.Cu" "B.Cu") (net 1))
 (via (at 147.828 87.884) (size 0.6) (drill 0.3) (layers "F.Cu" "B.Cu") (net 1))
 (via (at 148.59 100.707) (size 0.6) (drill 0.3) (layers "F.Cu" "B.Cu") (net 1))
 (via (at 146.304 111.506) (size 0.6) (drill 0.3) (layers "F.Cu" "B.Cu") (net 1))
 (segment (start 148.59 97.151) (end 146.562 97.151) (width 0.68) (layer "F.Cu") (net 4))
 (segment (start 150.575 97.151) (end 148.59 97.151) (width 0.68) (layer "F.Cu") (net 4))
 (segment (start 146.562 97.151) (end 146.558 97.155) (width 0.68) (layer "F.Cu") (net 4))
 (segment (start 151.4 97.976) (end 150.575 97.151) (width 0.2) (layer "F.Cu") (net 4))
 (segment (start 151.4 98.675) (end 151.4 97.976) (width 0.2) (layer "F.Cu") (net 4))
 (segment (start 145.161 93.091) (end 144.78 92.71) (width 0.2) (layer "F.Cu") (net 6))
 (segment (start 150.9 101.6) (end 150.9 102.338) (width 0.2) (layer "F.Cu") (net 6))
 (segment (start 140.97 89.789) (end 140.97 92.71) (width 0.2) (layer "F.Cu") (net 6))
 (segment (start 149.352 101.473) (end 145.669 101.473) (width 0.2) (layer "F.Cu") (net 6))
 (segment (start 150.9 102.338) (end 150.622 102.616) (width 0.2) (layer "F.Cu") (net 6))
 (segment (start 149.733 101.854) (end 149.352 101.473) (width 0.2) (layer "F.Cu") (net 6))
 (segment (start 145.669 101.473) (end 145.161 100.965) (width 0.2) (layer "F.Cu") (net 6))
 (segment (start 149.987 102.616) (end 149.733 102.362) (width 0.2) (layer "F.Cu") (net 6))
 (segment (start 150.622 102.616) (end 149.987 102.616) (width 0.2) (layer "F.Cu") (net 6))
 (segment (start 144.78 92.71) (end 140.97 92.71) (width 0.2) (layer "F.Cu") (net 6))
 (segment (start 149.733 102.362) (end 149.733 101.854) (width 0.2) (layer "F.Cu") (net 6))
 (segment (start 145.161 100.965) (end 145.161 93.091) (width 0.2) (layer "F.Cu") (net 6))
 (segment (start 152.4 87.63) (end 152.4 91.44) (width 0.68) (layer "F.Cu") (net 2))
 (segment (start 152.4 91.44) (end 152.4 93.341) (width 0.68) (layer "F.Cu") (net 2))
 (segment (start 152.4 97.151) (end 152.4 97.908704) (width 0.68) (layer "F.Cu") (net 3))
 (segment (start 152.4 98.675) (end 152.4 97.908704) (width 0.2) (layer "F.Cu") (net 3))
 (segment (start 152.4 95.416) (end 152.4 97.151) (width 0.68) (layer "F.Cu") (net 3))
 (segment (start 142.621 107.95) (end 143.256 107.315) (width 0.5) (layer "F.Cu") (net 12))
 (segment (start 143.764 105.918) (end 146.32 105.918) (width 0.5) (layer "F.Cu") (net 12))
 (segment (start 143.256 107.315) (end 143.256 106.426) (width 0.5) (layer "F.Cu") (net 12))
 (segment (start 143.256 106.426) (end 143.764 105.918) (width 0.5) (layer "F.Cu") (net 12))
 (segment (start 140.97 107.95) (end 142.621 107.95) (width 0.5) (layer "F.Cu") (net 12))
 (segment (start 150.876 103.124) (end 150.749 103.251) (width 0.2) (layer "F.Cu") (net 20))
 (segment (start 156.718 99.949) (end 156.718 98.409) (width 0.2) (layer "F.Cu") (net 20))
 (segment (start 150.749 103.251) (end 149.225 103.251) (width 0.2) (layer "F.Cu") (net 20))
 (segment (start 151.4 102.6) (end 150.876 103.124) (width 0.2) (layer "F.Cu") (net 20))
 (segment (start 151.4 101.6) (end 151.4 102.6) (width 0.2) (layer "F.Cu") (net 20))
 (via (at 149.225 103.251) (size 0.6) (drill 0.3) (layers "F.Cu" "B.Cu") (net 20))
 (via (at 156.718 99.949) (size 0.6) (drill 0.3) (layers "F.Cu" "B.Cu") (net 20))
 (segment (start 153.416 103.251) (end 156.718 99.949) (width 0.2) (layer "B.Cu") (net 20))
 (segment (start 149.225 103.251) (end 153.416 103.251) (width 0.2) (layer "B.Cu") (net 20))
 (segment (start 151.13 103.378) (end 150.506997 104.001003) (width 0.2) (layer "F.Cu") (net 21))
 (segment (start 151.9 102.608) (end 151.13 103.378) (width 0.2) (layer "F.Cu") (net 21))
 (segment (start 151.9 101.6) (end 151.9 102.608) (width 0.2) (layer "F.Cu") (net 21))
 (segment (start 158.623 99.949) (end 158.623 98.409) (width 0.2) (layer "F.Cu") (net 21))
 (segment (start 150.506997 104.001003) (end 149.225 104.001003) (width 0.2) (layer "F.Cu") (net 21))
 (via (at 158.623 99.949) (size 0.6) (drill 0.3) (layers "F.Cu" "B.Cu") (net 21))
 (via (at 149.225 104.001003) (size 0.6) (drill 0.3) (layers "F.Cu" "B.Cu") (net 21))
 (segment (start 149.225 104.001003) (end 154.570997 104.001003) (width 0.2) (layer "B.Cu") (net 21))
 (segment (start 154.570997 104.001003) (end 158.623 99.949) (width 0.2) (layer "B.Cu") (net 21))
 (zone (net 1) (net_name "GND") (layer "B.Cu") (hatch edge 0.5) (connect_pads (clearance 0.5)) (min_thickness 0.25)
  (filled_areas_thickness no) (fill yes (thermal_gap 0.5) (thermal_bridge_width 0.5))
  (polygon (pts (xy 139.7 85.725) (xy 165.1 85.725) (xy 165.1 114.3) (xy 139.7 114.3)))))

